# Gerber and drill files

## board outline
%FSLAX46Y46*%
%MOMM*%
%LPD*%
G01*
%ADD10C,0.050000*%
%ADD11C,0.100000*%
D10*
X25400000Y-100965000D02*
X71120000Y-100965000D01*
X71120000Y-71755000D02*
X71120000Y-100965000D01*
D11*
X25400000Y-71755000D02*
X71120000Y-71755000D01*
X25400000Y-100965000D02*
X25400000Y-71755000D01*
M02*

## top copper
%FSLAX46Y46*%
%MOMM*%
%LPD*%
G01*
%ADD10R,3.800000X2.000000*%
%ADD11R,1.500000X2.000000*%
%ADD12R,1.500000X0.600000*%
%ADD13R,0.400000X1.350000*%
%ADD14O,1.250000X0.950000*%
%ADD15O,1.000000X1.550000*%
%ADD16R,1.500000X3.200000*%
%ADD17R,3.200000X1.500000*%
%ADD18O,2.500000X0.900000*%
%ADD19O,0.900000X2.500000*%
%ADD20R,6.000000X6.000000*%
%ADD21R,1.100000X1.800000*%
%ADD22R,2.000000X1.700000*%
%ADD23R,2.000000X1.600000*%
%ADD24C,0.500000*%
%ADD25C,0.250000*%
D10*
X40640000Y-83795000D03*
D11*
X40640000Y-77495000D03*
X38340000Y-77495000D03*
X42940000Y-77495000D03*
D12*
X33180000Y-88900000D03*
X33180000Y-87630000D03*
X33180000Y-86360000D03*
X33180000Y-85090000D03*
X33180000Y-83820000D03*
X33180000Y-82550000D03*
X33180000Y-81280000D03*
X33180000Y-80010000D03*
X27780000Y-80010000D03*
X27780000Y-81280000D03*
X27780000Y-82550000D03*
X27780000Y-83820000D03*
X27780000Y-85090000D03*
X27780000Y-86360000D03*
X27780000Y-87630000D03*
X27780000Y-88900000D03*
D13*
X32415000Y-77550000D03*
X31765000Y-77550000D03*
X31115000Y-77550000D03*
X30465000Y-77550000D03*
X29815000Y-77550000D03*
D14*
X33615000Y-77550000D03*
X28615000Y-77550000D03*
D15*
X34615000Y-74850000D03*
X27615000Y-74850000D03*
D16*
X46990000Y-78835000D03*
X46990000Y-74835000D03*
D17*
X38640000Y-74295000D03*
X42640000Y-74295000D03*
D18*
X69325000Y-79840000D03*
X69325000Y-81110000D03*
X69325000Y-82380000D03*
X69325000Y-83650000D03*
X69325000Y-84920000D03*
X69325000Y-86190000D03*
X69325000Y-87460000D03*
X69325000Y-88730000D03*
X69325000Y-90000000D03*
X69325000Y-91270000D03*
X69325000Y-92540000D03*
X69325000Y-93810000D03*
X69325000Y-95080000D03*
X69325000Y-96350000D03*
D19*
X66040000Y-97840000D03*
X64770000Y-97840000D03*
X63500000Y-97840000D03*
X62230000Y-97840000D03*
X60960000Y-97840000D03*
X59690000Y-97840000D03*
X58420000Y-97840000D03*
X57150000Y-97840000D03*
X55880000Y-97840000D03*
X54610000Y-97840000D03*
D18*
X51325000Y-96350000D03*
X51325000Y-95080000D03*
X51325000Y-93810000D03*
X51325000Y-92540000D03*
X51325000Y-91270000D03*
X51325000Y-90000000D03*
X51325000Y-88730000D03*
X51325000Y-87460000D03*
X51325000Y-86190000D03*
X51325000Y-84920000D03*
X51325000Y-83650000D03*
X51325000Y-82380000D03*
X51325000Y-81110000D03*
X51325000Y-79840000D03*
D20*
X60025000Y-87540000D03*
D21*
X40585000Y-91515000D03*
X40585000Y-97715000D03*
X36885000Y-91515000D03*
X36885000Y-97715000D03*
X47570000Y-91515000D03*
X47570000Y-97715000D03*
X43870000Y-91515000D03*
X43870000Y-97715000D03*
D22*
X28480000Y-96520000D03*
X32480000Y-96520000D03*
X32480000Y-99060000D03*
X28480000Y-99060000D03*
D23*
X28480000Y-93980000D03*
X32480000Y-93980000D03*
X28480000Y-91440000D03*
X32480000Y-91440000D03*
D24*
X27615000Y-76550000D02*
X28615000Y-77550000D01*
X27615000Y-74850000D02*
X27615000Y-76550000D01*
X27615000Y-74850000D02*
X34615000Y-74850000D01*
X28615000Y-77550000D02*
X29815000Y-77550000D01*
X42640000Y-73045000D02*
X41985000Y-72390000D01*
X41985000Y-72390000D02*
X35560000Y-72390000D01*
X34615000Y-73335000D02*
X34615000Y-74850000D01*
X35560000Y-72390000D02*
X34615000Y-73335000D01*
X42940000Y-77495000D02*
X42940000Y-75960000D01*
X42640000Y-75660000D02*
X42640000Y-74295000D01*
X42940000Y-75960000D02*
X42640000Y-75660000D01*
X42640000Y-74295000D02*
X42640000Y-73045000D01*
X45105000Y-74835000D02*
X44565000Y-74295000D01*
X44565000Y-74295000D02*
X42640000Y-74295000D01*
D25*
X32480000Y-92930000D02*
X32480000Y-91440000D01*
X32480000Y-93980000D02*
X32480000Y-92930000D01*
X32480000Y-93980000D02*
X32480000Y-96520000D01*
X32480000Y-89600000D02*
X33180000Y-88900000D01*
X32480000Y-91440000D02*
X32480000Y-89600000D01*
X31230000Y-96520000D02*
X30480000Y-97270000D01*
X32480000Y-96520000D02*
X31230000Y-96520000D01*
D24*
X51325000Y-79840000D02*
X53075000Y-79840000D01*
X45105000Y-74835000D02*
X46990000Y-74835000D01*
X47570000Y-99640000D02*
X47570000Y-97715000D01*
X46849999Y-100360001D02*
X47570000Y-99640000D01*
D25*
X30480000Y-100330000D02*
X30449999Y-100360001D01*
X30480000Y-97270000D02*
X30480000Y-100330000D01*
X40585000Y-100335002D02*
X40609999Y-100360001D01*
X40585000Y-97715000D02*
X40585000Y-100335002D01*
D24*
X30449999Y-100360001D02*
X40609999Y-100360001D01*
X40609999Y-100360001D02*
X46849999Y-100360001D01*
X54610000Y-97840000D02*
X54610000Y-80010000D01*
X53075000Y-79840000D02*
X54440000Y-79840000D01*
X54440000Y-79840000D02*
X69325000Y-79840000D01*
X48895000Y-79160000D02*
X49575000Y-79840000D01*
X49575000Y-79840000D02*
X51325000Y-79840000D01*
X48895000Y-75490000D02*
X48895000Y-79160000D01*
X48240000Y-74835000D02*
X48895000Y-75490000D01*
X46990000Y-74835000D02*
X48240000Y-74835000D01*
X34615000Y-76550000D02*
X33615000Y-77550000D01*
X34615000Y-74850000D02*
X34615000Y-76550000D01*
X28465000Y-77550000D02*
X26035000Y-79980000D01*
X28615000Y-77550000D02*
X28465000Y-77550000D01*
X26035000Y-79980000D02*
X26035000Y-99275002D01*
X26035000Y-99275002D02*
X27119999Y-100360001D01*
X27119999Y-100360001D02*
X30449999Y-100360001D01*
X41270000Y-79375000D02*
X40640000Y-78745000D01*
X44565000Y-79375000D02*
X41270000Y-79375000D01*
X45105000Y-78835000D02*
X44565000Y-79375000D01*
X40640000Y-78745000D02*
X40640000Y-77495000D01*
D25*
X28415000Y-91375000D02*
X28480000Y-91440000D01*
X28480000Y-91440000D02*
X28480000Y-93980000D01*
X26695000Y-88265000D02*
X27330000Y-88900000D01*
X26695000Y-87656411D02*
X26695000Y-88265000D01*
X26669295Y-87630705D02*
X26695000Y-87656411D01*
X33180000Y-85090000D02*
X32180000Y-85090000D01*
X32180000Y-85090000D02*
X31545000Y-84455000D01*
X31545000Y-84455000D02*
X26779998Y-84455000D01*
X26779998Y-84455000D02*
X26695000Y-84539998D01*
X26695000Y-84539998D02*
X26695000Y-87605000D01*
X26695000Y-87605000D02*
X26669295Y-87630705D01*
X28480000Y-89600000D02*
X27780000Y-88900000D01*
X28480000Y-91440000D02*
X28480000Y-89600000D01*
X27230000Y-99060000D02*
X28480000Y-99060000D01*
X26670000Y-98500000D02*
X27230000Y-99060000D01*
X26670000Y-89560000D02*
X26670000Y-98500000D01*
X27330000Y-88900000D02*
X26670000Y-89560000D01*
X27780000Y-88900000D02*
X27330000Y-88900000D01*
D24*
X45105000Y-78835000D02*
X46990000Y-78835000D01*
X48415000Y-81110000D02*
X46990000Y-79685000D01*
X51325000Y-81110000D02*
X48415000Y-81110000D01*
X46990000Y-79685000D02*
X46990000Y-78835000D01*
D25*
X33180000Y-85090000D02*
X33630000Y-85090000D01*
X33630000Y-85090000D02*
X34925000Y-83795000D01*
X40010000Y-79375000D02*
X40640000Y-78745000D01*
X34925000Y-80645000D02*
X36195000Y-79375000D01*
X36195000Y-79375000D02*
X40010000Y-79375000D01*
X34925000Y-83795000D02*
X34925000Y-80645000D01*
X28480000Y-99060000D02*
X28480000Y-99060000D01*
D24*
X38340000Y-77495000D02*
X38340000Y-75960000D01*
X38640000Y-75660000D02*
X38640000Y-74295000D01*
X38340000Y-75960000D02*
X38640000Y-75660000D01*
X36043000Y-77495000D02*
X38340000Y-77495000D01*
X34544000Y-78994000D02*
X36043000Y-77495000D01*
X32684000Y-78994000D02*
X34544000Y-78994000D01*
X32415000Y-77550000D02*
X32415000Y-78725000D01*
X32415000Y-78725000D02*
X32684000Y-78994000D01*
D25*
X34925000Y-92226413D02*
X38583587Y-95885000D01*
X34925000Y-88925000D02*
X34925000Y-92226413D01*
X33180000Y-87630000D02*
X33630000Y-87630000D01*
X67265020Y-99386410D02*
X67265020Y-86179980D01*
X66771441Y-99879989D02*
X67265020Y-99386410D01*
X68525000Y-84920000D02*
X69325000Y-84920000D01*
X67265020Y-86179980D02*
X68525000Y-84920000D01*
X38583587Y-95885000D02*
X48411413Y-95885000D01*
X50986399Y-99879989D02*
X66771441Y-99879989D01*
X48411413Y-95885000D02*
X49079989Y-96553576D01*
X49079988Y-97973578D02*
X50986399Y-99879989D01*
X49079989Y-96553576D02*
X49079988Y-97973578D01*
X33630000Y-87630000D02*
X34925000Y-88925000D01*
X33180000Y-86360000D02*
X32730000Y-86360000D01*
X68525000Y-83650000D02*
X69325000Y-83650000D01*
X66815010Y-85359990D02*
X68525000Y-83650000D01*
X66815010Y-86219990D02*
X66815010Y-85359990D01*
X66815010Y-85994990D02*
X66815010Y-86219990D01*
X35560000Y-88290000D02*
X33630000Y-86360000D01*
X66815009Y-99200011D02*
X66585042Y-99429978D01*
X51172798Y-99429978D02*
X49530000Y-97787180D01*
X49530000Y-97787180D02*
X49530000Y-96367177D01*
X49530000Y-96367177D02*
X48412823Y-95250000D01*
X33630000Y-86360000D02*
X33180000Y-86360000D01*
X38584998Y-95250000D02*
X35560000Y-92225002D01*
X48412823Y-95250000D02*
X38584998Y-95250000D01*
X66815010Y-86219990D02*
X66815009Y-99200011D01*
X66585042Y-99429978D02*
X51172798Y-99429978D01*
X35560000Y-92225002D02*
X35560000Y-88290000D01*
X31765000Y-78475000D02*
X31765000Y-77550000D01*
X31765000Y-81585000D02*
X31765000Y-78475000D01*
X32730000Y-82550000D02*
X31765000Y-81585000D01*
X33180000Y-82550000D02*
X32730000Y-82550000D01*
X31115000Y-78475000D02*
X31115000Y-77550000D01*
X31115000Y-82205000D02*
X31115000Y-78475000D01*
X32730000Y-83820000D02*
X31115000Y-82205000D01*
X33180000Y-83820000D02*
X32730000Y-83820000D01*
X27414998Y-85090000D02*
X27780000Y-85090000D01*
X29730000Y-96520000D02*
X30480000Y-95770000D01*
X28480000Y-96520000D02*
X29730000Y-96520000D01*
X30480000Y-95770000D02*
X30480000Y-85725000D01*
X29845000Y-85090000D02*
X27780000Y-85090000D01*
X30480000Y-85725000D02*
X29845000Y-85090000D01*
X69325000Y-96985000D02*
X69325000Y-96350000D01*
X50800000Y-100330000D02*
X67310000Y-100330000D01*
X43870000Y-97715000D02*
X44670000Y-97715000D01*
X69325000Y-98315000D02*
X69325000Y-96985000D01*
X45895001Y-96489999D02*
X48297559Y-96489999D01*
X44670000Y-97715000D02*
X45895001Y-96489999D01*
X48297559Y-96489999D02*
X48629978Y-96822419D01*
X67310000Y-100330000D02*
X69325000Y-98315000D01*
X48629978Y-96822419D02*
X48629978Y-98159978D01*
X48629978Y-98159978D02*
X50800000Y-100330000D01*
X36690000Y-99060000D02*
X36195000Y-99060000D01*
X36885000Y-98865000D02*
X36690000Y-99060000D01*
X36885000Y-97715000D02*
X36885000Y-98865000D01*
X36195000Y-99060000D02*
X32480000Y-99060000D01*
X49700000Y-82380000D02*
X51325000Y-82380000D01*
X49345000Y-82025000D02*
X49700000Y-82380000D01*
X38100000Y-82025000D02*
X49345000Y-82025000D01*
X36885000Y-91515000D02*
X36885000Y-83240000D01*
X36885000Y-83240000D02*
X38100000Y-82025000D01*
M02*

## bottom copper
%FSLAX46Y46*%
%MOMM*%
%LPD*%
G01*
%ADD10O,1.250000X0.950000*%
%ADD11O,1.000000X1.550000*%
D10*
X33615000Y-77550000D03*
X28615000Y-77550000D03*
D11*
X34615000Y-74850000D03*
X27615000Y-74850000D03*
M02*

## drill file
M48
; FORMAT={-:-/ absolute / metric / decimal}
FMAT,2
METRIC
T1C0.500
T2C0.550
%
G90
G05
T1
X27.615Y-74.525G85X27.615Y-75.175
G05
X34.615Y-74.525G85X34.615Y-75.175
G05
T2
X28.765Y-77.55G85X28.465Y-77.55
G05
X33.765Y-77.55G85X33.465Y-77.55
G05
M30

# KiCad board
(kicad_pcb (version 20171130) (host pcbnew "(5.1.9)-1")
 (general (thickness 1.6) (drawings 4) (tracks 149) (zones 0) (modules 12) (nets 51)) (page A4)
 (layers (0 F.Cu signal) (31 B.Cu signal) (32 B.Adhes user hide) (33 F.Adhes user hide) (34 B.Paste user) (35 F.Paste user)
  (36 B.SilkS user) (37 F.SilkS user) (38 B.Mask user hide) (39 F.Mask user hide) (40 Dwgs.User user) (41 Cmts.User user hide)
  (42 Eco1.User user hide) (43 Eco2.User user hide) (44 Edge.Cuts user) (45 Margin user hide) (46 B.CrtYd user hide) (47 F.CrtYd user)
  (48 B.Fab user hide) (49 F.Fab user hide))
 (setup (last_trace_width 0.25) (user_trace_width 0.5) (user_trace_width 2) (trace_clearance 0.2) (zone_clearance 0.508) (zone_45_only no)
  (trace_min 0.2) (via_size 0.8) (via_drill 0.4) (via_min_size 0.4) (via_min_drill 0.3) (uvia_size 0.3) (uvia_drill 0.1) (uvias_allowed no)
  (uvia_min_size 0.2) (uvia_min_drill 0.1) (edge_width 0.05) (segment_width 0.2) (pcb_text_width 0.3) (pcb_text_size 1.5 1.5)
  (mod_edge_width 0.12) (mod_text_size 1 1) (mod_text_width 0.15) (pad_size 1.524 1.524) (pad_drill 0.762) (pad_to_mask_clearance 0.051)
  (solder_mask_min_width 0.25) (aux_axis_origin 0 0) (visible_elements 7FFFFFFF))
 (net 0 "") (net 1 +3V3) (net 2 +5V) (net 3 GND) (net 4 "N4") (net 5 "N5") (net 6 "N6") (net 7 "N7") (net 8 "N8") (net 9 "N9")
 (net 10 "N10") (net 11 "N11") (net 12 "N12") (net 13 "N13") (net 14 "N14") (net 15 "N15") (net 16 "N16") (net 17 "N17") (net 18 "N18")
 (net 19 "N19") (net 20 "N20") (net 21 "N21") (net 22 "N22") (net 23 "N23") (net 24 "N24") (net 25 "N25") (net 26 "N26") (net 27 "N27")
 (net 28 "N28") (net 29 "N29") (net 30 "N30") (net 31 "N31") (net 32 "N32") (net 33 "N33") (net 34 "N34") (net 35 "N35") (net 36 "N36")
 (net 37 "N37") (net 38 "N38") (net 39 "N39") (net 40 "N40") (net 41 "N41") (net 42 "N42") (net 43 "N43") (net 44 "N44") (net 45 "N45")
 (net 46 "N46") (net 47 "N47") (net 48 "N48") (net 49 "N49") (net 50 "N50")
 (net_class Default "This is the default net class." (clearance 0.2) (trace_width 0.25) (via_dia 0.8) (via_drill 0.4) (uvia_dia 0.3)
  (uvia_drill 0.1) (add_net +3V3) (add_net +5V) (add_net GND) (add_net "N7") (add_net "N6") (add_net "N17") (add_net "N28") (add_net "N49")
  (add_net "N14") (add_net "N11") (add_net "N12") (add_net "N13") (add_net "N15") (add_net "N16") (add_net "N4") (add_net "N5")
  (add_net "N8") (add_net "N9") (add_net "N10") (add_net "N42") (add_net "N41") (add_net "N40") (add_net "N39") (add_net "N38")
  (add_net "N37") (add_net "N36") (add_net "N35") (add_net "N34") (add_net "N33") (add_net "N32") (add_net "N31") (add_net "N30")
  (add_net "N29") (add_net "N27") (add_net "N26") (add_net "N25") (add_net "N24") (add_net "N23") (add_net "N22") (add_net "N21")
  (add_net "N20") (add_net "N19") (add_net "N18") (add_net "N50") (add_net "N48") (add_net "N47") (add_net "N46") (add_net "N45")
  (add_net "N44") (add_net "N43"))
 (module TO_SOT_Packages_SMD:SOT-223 (layer F.Cu) (at 40.64 80.645 270)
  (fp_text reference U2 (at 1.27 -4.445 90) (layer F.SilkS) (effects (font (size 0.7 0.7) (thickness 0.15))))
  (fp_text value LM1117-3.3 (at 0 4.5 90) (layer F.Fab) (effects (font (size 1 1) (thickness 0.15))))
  (pad 4 smd rect (at 3.15 0 270) (size 2 3.8) (layers F.Cu F.Paste F.Mask))
  (pad 2 smd rect (at -3.15 0 270) (size 2 1.5) (layers F.Cu F.Paste F.Mask) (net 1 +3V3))
  (pad 3 smd rect (at -3.15 2.3 270) (size 2 1.5) (layers F.Cu F.Paste F.Mask) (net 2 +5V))
  (pad 1 smd rect (at -3.15 -2.3 270) (size 2 1.5) (layers F.Cu F.Paste F.Mask) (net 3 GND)))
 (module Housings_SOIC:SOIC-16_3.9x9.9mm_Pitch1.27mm (layer F.Cu) (at 30.48 84.455 180)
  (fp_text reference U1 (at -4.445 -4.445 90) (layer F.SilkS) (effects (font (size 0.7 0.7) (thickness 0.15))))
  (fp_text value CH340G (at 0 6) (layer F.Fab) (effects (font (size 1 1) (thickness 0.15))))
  (pad 1 smd rect (at -2.7 -4.445 180) (size 1.5 0.6) (layers F.Cu F.Paste F.Mask) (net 3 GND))
  (pad 2 smd rect (at -2.7 -3.175 180) (size 1.5 0.6) (layers F.Cu F.Paste F.Mask) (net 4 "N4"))
  (pad 3 smd rect (at -2.7 -1.905 180) (size 1.5 0.6) (layers F.Cu F.Paste F.Mask) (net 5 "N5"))
  (pad 4 smd rect (at -2.7 -0.635 180) (size 1.5 0.6) (layers F.Cu F.Paste F.Mask) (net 1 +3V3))
  (pad 5 smd rect (at -2.7 0.635 180) (size 1.5 0.6) (layers F.Cu F.Paste F.Mask) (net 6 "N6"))
  (pad 6 smd rect (at -2.7 1.905 180) (size 1.5 0.6) (layers F.Cu F.Paste F.Mask) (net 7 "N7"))
  (pad 7 smd rect (at -2.7 3.175 180) (size 1.5 0.6) (layers F.Cu F.Paste F.Mask) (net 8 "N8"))
  (pad 8 smd rect (at -2.7 4.445 180) (size 1.5 0.6) (layers F.Cu F.Paste F.Mask) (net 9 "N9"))
  (pad 9 smd rect (at 2.7 4.445 180) (size 1.5 0.6) (layers F.Cu F.Paste F.Mask) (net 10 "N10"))
  (pad 10 smd rect (at 2.7 3.175 180) (size 1.5 0.6) (layers F.Cu F.Paste F.Mask) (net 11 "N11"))
  (pad 11 smd rect (at 2.7 1.905 180) (size 1.5 0.6) (layers F.Cu F.Paste F.Mask) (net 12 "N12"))
  (pad 12 smd rect (at 2.7 0.635 180) (size 1.5 0.6) (layers F.Cu F.Paste F.Mask) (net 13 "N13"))
  (pad 13 smd rect (at 2.7 -0.635 180) (size 1.5 0.6) (layers F.Cu F.Paste F.Mask) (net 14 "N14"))
  (pad 14 smd rect (at 2.7 -1.905 180) (size 1.5 0.6) (layers F.Cu F.Paste F.Mask) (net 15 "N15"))
  (pad 15 smd rect (at 2.7 -3.175 180) (size 1.5 0.6) (layers F.Cu F.Paste F.Mask) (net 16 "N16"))
  (pad 16 smd rect (at 2.7 -4.445 180) (size 1.5 0.6) (layers F.Cu F.Paste F.Mask) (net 1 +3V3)))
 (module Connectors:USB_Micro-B (layer F.Cu) (at 31.115 76.2 180)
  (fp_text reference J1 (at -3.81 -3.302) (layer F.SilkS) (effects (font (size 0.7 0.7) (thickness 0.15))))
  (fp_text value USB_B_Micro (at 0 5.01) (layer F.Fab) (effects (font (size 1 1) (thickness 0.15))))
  (pad 1 smd rect (at -1.3 -1.35 270) (size 1.35 0.4) (layers F.Cu F.Paste F.Mask) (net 2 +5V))
  (pad 2 smd rect (at -0.65 -1.35 270) (size 1.35 0.4) (layers F.Cu F.Paste F.Mask) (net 7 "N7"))
  (pad 3 smd rect (at 0 -1.35 270) (size 1.35 0.4) (layers F.Cu F.Paste F.Mask) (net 6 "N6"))
  (pad 4 smd rect (at 0.65 -1.35 270) (size 1.35 0.4) (layers F.Cu F.Paste F.Mask) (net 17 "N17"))
  (pad 5 smd rect (at 1.3 -1.35 270) (size 1.35 0.4) (layers F.Cu F.Paste F.Mask) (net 3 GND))
  (pad 6 thru_hole oval (at -2.5 -1.35 270) (size 0.95 1.25) (drill oval 0.55 0.85) (layers *.Cu *.Mask) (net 3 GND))
  (pad 6 thru_hole oval (at 2.5 -1.35 270) (size 0.95 1.25) (drill oval 0.55 0.85) (layers *.Cu *.Mask) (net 3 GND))
  (pad 6 thru_hole oval (at -3.5 1.35 270) (size 1.55 1) (drill oval 1.15 0.5) (layers *.Cu *.Mask) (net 3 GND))
  (pad 6 thru_hole oval (at 3.5 1.35 270) (size 1.55 1) (drill oval 1.15 0.5) (layers *.Cu *.Mask) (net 3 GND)))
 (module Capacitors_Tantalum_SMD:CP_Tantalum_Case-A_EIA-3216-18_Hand (layer F.Cu) (at 46.99 76.835 90)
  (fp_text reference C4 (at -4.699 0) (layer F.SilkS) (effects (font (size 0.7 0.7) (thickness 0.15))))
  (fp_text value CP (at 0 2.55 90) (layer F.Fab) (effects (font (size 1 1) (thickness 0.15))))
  (pad 1 smd rect (at -2 0 90) (size 3.2 1.5) (layers F.Cu F.Paste F.Mask) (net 1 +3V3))
  (pad 2 smd rect (at 2 0 90) (size 3.2 1.5) (layers F.Cu F.Paste F.Mask) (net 3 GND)))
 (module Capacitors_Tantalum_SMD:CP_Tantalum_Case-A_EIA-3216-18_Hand (layer F.Cu) (at 40.64 74.295)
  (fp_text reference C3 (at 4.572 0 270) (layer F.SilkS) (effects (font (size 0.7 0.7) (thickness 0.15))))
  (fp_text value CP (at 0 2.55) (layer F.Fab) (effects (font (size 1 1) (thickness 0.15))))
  (pad 1 smd rect (at -2 0) (size 3.2 1.5) (layers F.Cu F.Paste F.Mask) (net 2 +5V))
  (pad 2 smd rect (at 2 0) (size 3.2 1.5) (layers F.Cu F.Paste F.Mask) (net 3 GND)))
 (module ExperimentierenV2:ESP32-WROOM (layer F.Cu) (at 60.325 85.09 180)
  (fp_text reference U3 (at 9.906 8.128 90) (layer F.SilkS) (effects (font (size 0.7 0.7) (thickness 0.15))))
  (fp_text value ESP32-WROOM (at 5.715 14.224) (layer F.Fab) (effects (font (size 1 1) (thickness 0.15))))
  (pad 38 smd oval (at -9 5.25 180) (size 2.5 0.9) (layers F.Cu F.Paste F.Mask) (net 3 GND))
  (pad 37 smd oval (at -9 3.98 180) (size 2.5 0.9) (layers F.Cu F.Paste F.Mask) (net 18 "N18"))
  (pad 36 smd oval (at -9 2.71 180) (size 2.5 0.9) (layers F.Cu F.Paste F.Mask) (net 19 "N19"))
  (pad 35 smd oval (at -9 1.44 180) (size 2.5 0.9) (layers F.Cu F.Paste F.Mask) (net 5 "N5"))
  (pad 34 smd oval (at -9 0.17 180) (size 2.5 0.9) (layers F.Cu F.Paste F.Mask) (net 4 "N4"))
  (pad 33 smd oval (at -9 -1.1 180) (size 2.5 0.9) (layers F.Cu F.Paste F.Mask) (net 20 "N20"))
  (pad 32 smd oval (at -9 -2.37 180) (size 2.5 0.9) (layers F.Cu F.Paste F.Mask) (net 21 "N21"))
  (pad 31 smd oval (at -9 -3.64 180) (size 2.5 0.9) (layers F.Cu F.Paste F.Mask) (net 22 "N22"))
  (pad 30 smd oval (at -9 -4.91 180) (size 2.5 0.9) (layers F.Cu F.Paste F.Mask) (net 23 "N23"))
  (pad 29 smd oval (at -9 -6.18 180) (size 2.5 0.9) (layers F.Cu F.Paste F.Mask) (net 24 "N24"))
  (pad 28 smd oval (at -9 -7.45 180) (size 2.5 0.9) (layers F.Cu F.Paste F.Mask) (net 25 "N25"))
  (pad 27 smd oval (at -9 -8.72 180) (size 2.5 0.9) (layers F.Cu F.Paste F.Mask) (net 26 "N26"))
  (pad 26 smd oval (at -9 -9.99 180) (size 2.5 0.9) (layers F.Cu F.Paste F.Mask) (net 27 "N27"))
  (pad 25 smd oval (at -9 -11.26 180) (size 2.5 0.9) (layers F.Cu F.Paste F.Mask) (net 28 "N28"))
  (pad 24 smd oval (at -5.715 -12.75 180) (size 0.9 2.5) (layers F.Cu F.Paste F.Mask) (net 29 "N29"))
  (pad 23 smd oval (at -4.445 -12.75 180) (size 0.9 2.5) (layers F.Cu F.Paste F.Mask) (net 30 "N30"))
  (pad 22 smd oval (at -3.175 -12.75 180) (size 0.9 2.5) (layers F.Cu F.Paste F.Mask) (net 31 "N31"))
  (pad 21 smd oval (at -1.905 -12.75 180) (size 0.9 2.5) (layers F.Cu F.Paste F.Mask) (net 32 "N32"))
  (pad 20 smd oval (at -0.635 -12.75 180) (size 0.9 2.5) (layers F.Cu F.Paste F.Mask) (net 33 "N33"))
  (pad 19 smd oval (at 0.635 -12.75 180) (size 0.9 2.5) (layers F.Cu F.Paste F.Mask) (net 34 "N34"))
  (pad 18 smd oval (at 1.905 -12.75 180) (size 0.9 2.5) (layers F.Cu F.Paste F.Mask) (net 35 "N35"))
  (pad 17 smd oval (at 3.175 -12.75 180) (size 0.9 2.5) (layers F.Cu F.Paste F.Mask) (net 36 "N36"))
  (pad 16 smd oval (at 4.445 -12.75 180) (size 0.9 2.5) (layers F.Cu F.Paste F.Mask) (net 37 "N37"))
  (pad 15 smd oval (at 5.715 -12.75 180) (size 0.9 2.5) (layers F.Cu F.Paste F.Mask) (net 3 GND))
  (pad 14 smd oval (at 9 -11.26 180) (size 2.5 0.9) (layers F.Cu F.Paste F.Mask) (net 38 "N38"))
  (pad 13 smd oval (at 9 -9.99 180) (size 2.5 0.9) (layers F.Cu F.Paste F.Mask) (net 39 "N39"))
  (pad 12 smd oval (at 9 -8.72 180) (size 2.5 0.9) (layers F.Cu F.Paste F.Mask) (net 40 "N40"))
  (pad 11 smd oval (at 9 -7.45 180) (size 2.5 0.9) (layers F.Cu F.Paste F.Mask) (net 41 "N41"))
  (pad 10 smd oval (at 9 -6.18 180) (size 2.5 0.9) (layers F.Cu F.Paste F.Mask) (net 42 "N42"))
  (pad 9 smd oval (at 9 -4.91 180) (size 2.5 0.9) (layers F.Cu F.Paste F.Mask) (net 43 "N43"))
  (pad 8 smd oval (at 9 -3.64 180) (size 2.5 0.9) (layers F.Cu F.Paste F.Mask) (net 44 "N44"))
  (pad 7 smd oval (at 9 -2.37 180) (size 2.5 0.9) (layers F.Cu F.Paste F.Mask) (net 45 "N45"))
  (pad 6 smd oval (at 9 -1.1 180) (size 2.5 0.9) (layers F.Cu F.Paste F.Mask) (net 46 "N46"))
  (pad 5 smd oval (at 9 0.17 180) (size 2.5 0.9) (layers F.Cu F.Paste F.Mask) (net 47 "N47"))
  (pad 4 smd oval (at 9 1.44 180) (size 2.5 0.9) (layers F.Cu F.Paste F.Mask) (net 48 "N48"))
  (pad 3 smd oval (at 9 2.71 180) (size 2.5 0.9) (layers F.Cu F.Paste F.Mask) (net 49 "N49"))
  (pad 2 smd oval (at 9 3.98 180) (size 2.5 0.9) (layers F.Cu F.Paste F.Mask) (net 1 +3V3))
  (pad 1 smd oval (at 9 5.25 180) (size 2.5 0.9) (layers F.Cu F.Paste F.Mask) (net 3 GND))
  (pad 39 smd rect (at 0.3 -2.45 180) (size 6 6) (layers F.Cu F.Paste F.Mask) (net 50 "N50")))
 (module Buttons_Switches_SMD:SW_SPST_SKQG (layer F.Cu) (at 38.735 94.615 270)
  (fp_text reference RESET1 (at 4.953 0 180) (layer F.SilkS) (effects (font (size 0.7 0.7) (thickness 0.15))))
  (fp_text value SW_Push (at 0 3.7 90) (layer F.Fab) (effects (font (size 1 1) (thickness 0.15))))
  (pad 1 smd rect (at -3.1 -1.85 270) (size 1.8 1.1) (layers F.Cu F.Paste F.Mask) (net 3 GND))
  (pad 1 smd rect (at 3.1 -1.85 270) (size 1.8 1.1) (layers F.Cu F.Paste F.Mask) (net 3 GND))
  (pad 2 smd rect (at -3.1 1.85 270) (size 1.8 1.1) (layers F.Cu F.Paste F.Mask) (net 49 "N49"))
  (pad 2 smd rect (at 3.1 1.85 270) (size 1.8 1.1) (layers F.Cu F.Paste F.Mask) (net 49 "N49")))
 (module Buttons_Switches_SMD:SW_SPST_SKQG (layer F.Cu) (at 45.72 94.615 270)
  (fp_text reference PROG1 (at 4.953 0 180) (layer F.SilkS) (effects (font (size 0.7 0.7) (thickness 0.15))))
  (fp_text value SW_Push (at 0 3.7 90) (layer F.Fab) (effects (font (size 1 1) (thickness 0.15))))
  (pad 1 smd rect (at -3.1 -1.85 270) (size 1.8 1.1) (layers F.Cu F.Paste F.Mask) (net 3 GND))
  (pad 1 smd rect (at 3.1 -1.85 270) (size 1.8 1.1) (layers F.Cu F.Paste F.Mask) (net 3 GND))
  (pad 2 smd rect (at -3.1 1.85 270) (size 1.8 1.1) (layers F.Cu F.Paste F.Mask) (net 28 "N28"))
  (pad 2 smd rect (at 3.1 1.85 270) (size 1.8 1.1) (layers F.Cu F.Paste F.Mask) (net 28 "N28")))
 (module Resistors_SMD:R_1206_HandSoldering (layer F.Cu) (at 30.48 96.52)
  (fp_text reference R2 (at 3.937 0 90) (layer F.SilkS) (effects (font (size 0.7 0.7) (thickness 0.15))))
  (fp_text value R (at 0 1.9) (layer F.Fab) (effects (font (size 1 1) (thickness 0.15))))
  (pad 1 smd rect (at -2 0) (size 2 1.7) (layers F.Cu F.Paste F.Mask) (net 14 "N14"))
  (pad 2 smd rect (at 2 0) (size 2 1.7) (layers F.Cu F.Paste F.Mask) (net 3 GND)))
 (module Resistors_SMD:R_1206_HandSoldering (layer F.Cu) (at 30.48 99.06 180)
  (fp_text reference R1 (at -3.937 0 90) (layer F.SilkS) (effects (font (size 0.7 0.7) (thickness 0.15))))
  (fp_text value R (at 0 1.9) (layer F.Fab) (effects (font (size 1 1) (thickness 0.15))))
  (pad 1 smd rect (at -2 0 180) (size 2 1.7) (layers F.Cu F.Paste F.Mask) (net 49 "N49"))
  (pad 2 smd rect (at 2 0 180) (size 2 1.7) (layers F.Cu F.Paste F.Mask) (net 1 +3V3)))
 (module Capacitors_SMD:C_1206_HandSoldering (layer F.Cu) (at 30.48 93.98)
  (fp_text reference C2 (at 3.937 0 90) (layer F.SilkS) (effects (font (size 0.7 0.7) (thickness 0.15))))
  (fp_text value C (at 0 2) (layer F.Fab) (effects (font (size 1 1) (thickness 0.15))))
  (pad 1 smd rect (at -2 0) (size 2 1.6) (layers F.Cu F.Paste F.Mask) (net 1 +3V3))
  (pad 2 smd rect (at 2 0) (size 2 1.6) (layers F.Cu F.Paste F.Mask) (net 3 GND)))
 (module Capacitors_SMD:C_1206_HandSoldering (layer F.Cu) (at 30.48 91.44)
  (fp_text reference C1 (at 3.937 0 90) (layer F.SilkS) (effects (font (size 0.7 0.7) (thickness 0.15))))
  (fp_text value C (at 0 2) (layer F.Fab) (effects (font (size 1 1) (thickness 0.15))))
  (pad 1 smd rect (at -2 0) (size 2 1.6) (layers F.Cu F.Paste F.Mask) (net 1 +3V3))
  (pad 2 smd rect (at 2 0) (size 2 1.6) (layers F.Cu F.Paste F.Mask) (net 3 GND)))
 (gr_line (start 25.4 100.965) (end 71.12 100.965) (layer Edge.Cuts) (width 0.05))
 (gr_line (start 71.12 71.755) (end 71.12 100.965) (layer Edge.Cuts) (width 0.05))
 (gr_line (start 25.4 71.755) (end 71.12 71.755) (layer Edge.Cuts) (width 0.1))
 (gr_line (start 25.4 100.965) (end 25.4 71.755) (layer Edge.Cuts) (width 0.1))
 (segment (start 27.615 76.55) (end 28.615 77.55) (width 0.5) (layer F.Cu) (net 3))
 (segment (start 27.615 74.85) (end 27.615 76.55) (width 0.5) (layer F.Cu) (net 3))
 (segment (start 27.615 74.85) (end 34.615 74.85) (width 0.5) (layer F.Cu) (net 3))
 (segment (start 28.615 77.55) (end 29.815 77.55) (width 0.5) (layer F.Cu) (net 3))
 (segment (start 42.64 73.045) (end 41.985 72.39) (width 0.5) (layer F.Cu) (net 3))
 (segment (start 41.985 72.39) (end 35.56 72.39) (width 0.5) (layer F.Cu) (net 3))
 (segment (start 34.615 73.335) (end 34.615 74.85) (width 0.5) (layer F.Cu) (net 3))
 (segment (start 35.56 72.39) (end 34.615 73.335) (width 0.5) (layer F.Cu) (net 3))
 (segment (start 42.94 77.495) (end 42.94 75.96) (width 0.5) (layer F.Cu) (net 3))
 (segment (start 42.64 75.66) (end 42.64 74.295) (width 0.5) (layer F.Cu) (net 3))
 (segment (start 42.94 75.96) (end 42.64 75.66) (width 0.5) (layer F.Cu) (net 3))
 (segment (start 42.64 74.295) (end 42.64 73.045) (width 0.5) (layer F.Cu) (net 3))
 (segment (start 45.105 74.835) (end 44.565 74.295) (width 0.5) (layer F.Cu) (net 3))
 (segment (start 44.565 74.295) (end 42.64 74.295) (width 0.5) (layer F.Cu) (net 3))
 (segment (start 32.48 92.93) (end 32.48 91.44) (width 0.25) (layer F.Cu) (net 3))
 (segment (start 32.48 93.98) (end 32.48 92.93) (width 0.25) (layer F.Cu) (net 3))
 (segment (start 32.48 93.98) (end 32.48 96.52) (width 0.25) (layer F.Cu) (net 3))
 (segment (start 32.48 89.6) (end 33.18 88.9) (width 0.25) (layer F.Cu) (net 3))
 (segment (start 32.48 91.44) (end 32.48 89.6) (width 0.25) (layer F.Cu) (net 3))
 (segment (start 31.23 96.52) (end 30.48 97.27) (width 0.25) (layer F.Cu) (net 3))
 (segment (start 32.48 96.52) (end 31.23 96.52) (width 0.25) (layer F.Cu) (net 3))
 (segment (start 51.325 79.84) (end 53.075 79.84) (width 0.5) (layer F.Cu) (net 3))
 (segment (start 45.105 74.835) (end 46.99 74.835) (width 0.5) (layer F.Cu) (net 3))
 (segment (start 47.57 99.64) (end 47.57 97.715) (width 0.5) (layer F.Cu) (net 3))
 (segment (start 46.849999 100.360001) (end 47.57 99.64) (width 0.5) (layer F.Cu) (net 3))
 (segment (start 30.48 100.33) (end 30.449999 100.360001) (width 0.25) (layer F.Cu) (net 3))
 (segment (start 30.48 97.27) (end 30.48 100.33) (width 0.25) (layer F.Cu) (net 3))
 (segment (start 40.585 100.335002) (end 40.609999 100.360001) (width 0.25) (layer F.Cu) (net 3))
 (segment (start 40.585 97.715) (end 40.585 100.335002) (width 0.25) (layer F.Cu) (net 3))
 (segment (start 30.449999 100.360001) (end 40.609999 100.360001) (width 0.5) (layer F.Cu) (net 3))
 (segment (start 40.609999 100.360001) (end 46.849999 100.360001) (width 0.5) (layer F.Cu) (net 3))
 (segment (start 54.61 97.84) (end 54.61 80.01) (width 0.5) (layer F.Cu) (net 3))
 (segment (start 53.075 79.84) (end 54.44 79.84) (width 0.5) (layer F.Cu) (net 3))
 (segment (start 54.44 79.84) (end 69.325 79.84) (width 0.5) (layer F.Cu) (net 3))
 (segment (start 48.895 79.16) (end 49.575 79.84) (width 0.5) (layer F.Cu) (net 3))
 (segment (start 49.575 79.84) (end 51.325 79.84) (width 0.5) (layer F.Cu) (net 3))
 (segment (start 48.895 75.49) (end 48.895 79.16) (width 0.5) (layer F.Cu) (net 3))
 (segment (start 48.24 74.835) (end 48.895 75.49) (width 0.5) (layer F.Cu) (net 3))
 (segment (start 46.99 74.835) (end 48.24 74.835) (width 0.5) (layer F.Cu) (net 3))
 (segment (start 34.615 76.55) (end 33.615 77.55) (width 0.5) (layer F.Cu) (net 3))
 (segment (start 34.615 74.85) (end 34.615 76.55) (width 0.5) (layer F.Cu) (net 3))
 (segment (start 28.465 77.55) (end 26.035 79.98) (width 0.5) (layer F.Cu) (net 3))
 (segment (start 28.615 77.55) (end 28.465 77.55) (width 0.5) (layer F.Cu) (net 3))
 (segment (start 26.035 79.98) (end 26.035 99.275002) (width 0.5) (layer F.Cu) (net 3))
 (segment (start 26.035 99.275002) (end 27.119999 100.360001) (width 0.5) (layer F.Cu) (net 3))
 (segment (start 27.119999 100.360001) (end 30.449999 100.360001) (width 0.5) (layer F.Cu) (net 3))
 (segment (start 41.27 79.375) (end 40.64 78.745) (width 0.5) (layer F.Cu) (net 1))
 (segment (start 44.565 79.375) (end 41.27 79.375) (width 0.5) (layer F.Cu) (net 1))
 (segment (start 45.105 78.835) (end 44.565 79.375) (width 0.5) (layer F.Cu) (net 1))
 (segment (start 40.64 78.745) (end 40.64 77.495) (width 0.5) (layer F.Cu) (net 1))
 (segment (start 28.415 91.375) (end 28.48 91.44) (width 0.25) (layer F.Cu) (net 1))
 (segment (start 28.48 91.44) (end 28.48 93.98) (width 0.25) (layer F.Cu) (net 1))
 (segment (start 26.695 88.265) (end 27.33 88.9) (width 0.25) (layer F.Cu) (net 1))
 (segment (start 26.695 87.656411) (end 26.695 88.265) (width 0.25) (layer F.Cu) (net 1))
 (segment (start 26.669295 87.630705) (end 26.695 87.656411) (width 0.25) (layer F.Cu) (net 1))
 (segment (start 33.18 85.09) (end 32.18 85.09) (width 0.25) (layer F.Cu) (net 1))
 (segment (start 32.18 85.09) (end 31.545 84.455) (width 0.25) (layer F.Cu) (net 1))
 (segment (start 31.545 84.455) (end 26.779998 84.455) (width 0.25) (layer F.Cu) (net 1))
 (segment (start 26.779998 84.455) (end 26.695 84.539998) (width 0.25) (layer F.Cu) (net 1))
 (segment (start 26.695 84.539998) (end 26.695 87.605) (width 0.25) (layer F.Cu) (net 1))
 (segment (start 26.695 87.605) (end 26.669295 87.630705) (width 0.25) (layer F.Cu) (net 1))
 (segment (start 28.48 89.6) (end 27.78 88.9) (width 0.25) (layer F.Cu) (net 1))
 (segment (start 28.48 91.44) (end 28.48 89.6) (width 0.25) (layer F.Cu) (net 1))
 (segment (start 27.23 99.06) (end 28.48 99.06) (width 0.25) (layer F.Cu) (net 1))
 (segment (start 26.67 98.5) (end 27.23 99.06) (width 0.25) (layer F.Cu) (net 1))
 (segment (start 26.67 89.56) (end 26.67 98.5) (width 0.25) (layer F.Cu) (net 1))
 (segment (start 27.33 88.9) (end 26.67 89.56) (width 0.25) (layer F.Cu) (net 1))
 (segment (start 27.78 88.9) (end 27.33 88.9) (width 0.25) (layer F.Cu) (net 1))
 (segment (start 45.105 78.835) (end 46.99 78.835) (width 0.5) (layer F.Cu) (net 1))
 (segment (start 48.415 81.11) (end 46.99 79.685) (width 0.5) (layer F.Cu) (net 1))
 (segment (start 51.325 81.11) (end 48.415 81.11) (width 0.5) (layer F.Cu) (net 1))
 (segment (start 46.99 79.685) (end 46.99 78.835) (width 0.5) (layer F.Cu) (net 1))
 (segment (start 33.18 85.09) (end 33.63 85.09) (width 0.25) (layer F.Cu) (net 1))
 (segment (start 33.63 85.09) (end 34.925 83.795) (width 0.25) (layer F.Cu) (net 1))
 (segment (start 40.01 79.375) (end 40.64 78.745) (width 0.25) (layer F.Cu) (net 1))
 (segment (start 34.925 80.645) (end 36.195 79.375) (width 0.25) (layer F.Cu) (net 1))
 (segment (start 36.195 79.375) (end 40.01 79.375) (width 0.25) (layer F.Cu) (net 1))
 (segment (start 34.925 83.795) (end 34.925 80.645) (width 0.25) (layer F.Cu) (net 1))
 (segment (start 28.48 99.06) (end 28.48 99.06) (width 0.25) (layer F.Cu) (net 1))
 (segment (start 38.34 77.495) (end 38.34 75.96) (width 0.5) (layer F.Cu) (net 2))
 (segment (start 38.64 75.66) (end 38.64 74.295) (width 0.5) (layer F.Cu) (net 2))
 (segment (start 38.34 75.96) (end 38.64 75.66) (width 0.5) (layer F.Cu) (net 2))
 (segment (start 36.043 77.495) (end 38.34 77.495) (width 0.5) (layer F.Cu) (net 2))
 (segment (start 34.544 78.994) (end 36.043 77.495) (width 0.5) (layer F.Cu) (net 2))
 (segment (start 32.684 78.994) (end 34.544 78.994) (width 0.5) (layer F.Cu) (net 2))
 (segment (start 32.415 77.55) (end 32.415 78.725) (width 0.5) (layer F.Cu) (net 2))
 (segment (start 32.415 78.725) (end 32.684 78.994) (width 0.5) (layer F.Cu) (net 2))
 (segment (start 34.925 92.226413) (end 38.583587 95.885) (width 0.25) (layer F.Cu) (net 4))
 (segment (start 34.925 88.925) (end 34.925 92.226413) (width 0.25) (layer F.Cu) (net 4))
 (segment (start 33.18 87.63) (end 33.63 87.63) (width 0.25) (layer F.Cu) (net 4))
 (segment (start 67.26502 99.38641) (end 67.26502 86.17998) (width 0.25) (layer F.Cu) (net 4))
 (segment (start 66.771441 99.879989) (end 67.26502 99.38641) (width 0.25) (layer F.Cu) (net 4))
 (segment (start 68.525 84.92) (end 69.325 84.92) (width 0.25) (layer F.Cu) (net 4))
 (segment (start 67.26502 86.17998) (end 68.525 84.92) (width 0.25) (layer F.Cu) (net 4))
 (segment (start 38.583587 95.885) (end 48.411413 95.885) (width 0.25) (layer F.Cu) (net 4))
 (segment (start 50.986399 99.879989) (end 66.771441 99.879989) (width 0.25) (layer F.Cu) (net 4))
 (segment (start 48.411413 95.885) (end 49.079989 96.553576) (width 0.25) (layer F.Cu) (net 4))
 (segment (start 49.079988 97.973578) (end 50.986399 99.879989) (width 0.25) (layer F.Cu) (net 4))
 (segment (start 49.079989 96.553576) (end 49.079988 97.973578) (width 0.25) (layer F.Cu) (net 4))
 (segment (start 33.63 87.63) (end 34.925 88.925) (width 0.25) (layer F.Cu) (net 4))
 (segment (start 33.18 86.36) (end 32.73 86.36) (width 0.25) (layer F.Cu) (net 5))
 (segment (start 68.525 83.65) (end 69.325 83.65) (width 0.25) (layer F.Cu) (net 5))
 (segment (start 66.81501 85.35999) (end 68.525 83.65) (width 0.25) (layer F.Cu) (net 5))
 (segment (start 66.81501 86.21999) (end 66.81501 85.35999) (width 0.25) (layer F.Cu) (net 5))
 (segment (start 66.81501 85.99499) (end 66.81501 86.21999) (width 0.25) (layer F.Cu) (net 5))
 (segment (start 35.56 88.29) (end 33.63 86.36) (width 0.25) (layer F.Cu) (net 5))
 (segment (start 66.815009 99.200011) (end 66.585042 99.429978) (width 0.25) (layer F.Cu) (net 5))
 (segment (start 51.172798 99.429978) (end 49.53 97.78718) (width 0.25) (layer F.Cu) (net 5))
 (segment (start 49.53 97.78718) (end 49.53 96.367177) (width 0.25) (layer F.Cu) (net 5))
 (segment (start 49.53 96.367177) (end 48.412823 95.25) (width 0.25) (layer F.Cu) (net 5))
 (segment (start 33.63 86.36) (end 33.18 86.36) (width 0.25) (layer F.Cu) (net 5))
 (segment (start 38.584998 95.25) (end 35.56 92.225002) (width 0.25) (layer F.Cu) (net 5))
 (segment (start 48.412823 95.25) (end 38.584998 95.25) (width 0.25) (layer F.Cu) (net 5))
 (segment (start 66.81501 86.21999) (end 66.815009 99.200011) (width 0.25) (layer F.Cu) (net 5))
 (segment (start 66.585042 99.429978) (end 51.172798 99.429978) (width 0.25) (layer F.Cu) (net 5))
 (segment (start 35.56 92.225002) (end 35.56 88.29) (width 0.25) (layer F.Cu) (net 5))
 (segment (start 31.765 78.475) (end 31.765 77.55) (width 0.25) (layer F.Cu) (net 7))
 (segment (start 31.765 81.585) (end 31.765 78.475) (width 0.25) (layer F.Cu) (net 7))
 (segment (start 32.73 82.55) (end 31.765 81.585) (width 0.25) (layer F.Cu) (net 7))
 (segment (start 33.18 82.55) (end 32.73 82.55) (width 0.25) (layer F.Cu) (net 7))
 (segment (start 31.115 78.475) (end 31.115 77.55) (width 0.25) (layer F.Cu) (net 6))
 (segment (start 31.115 82.205) (end 31.115 78.475) (width 0.25) (layer F.Cu) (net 6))
 (segment (start 32.73 83.82) (end 31.115 82.205) (width 0.25) (layer F.Cu) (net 6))
 (segment (start 33.18 83.82) (end 32.73 83.82) (width 0.25) (layer F.Cu) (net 6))
 (segment (start 27.414998 85.09) (end 27.78 85.09) (width 0.25) (layer F.Cu) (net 14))
 (segment (start 29.73 96.52) (end 30.48 95.77) (width 0.25) (layer F.Cu) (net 14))
 (segment (start 28.48 96.52) (end 29.73 96.52) (width 0.25) (layer F.Cu) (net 14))
 (segment (start 30.48 95.77) (end 30.48 85.725) (width 0.25) (layer F.Cu) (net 14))
 (segment (start 29.845 85.09) (end 27.78 85.09) (width 0.25) (layer F.Cu) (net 14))
 (segment (start 30.48 85.725) (end 29.845 85.09) (width 0.25) (layer F.Cu) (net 14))
 (segment (start 69.325 96.985) (end 69.325 96.35) (width 0.25) (layer F.Cu) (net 28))
 (segment (start 50.8 100.33) (end 67.31 100.33) (width 0.25) (layer F.Cu) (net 28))
 (segment (start 43.87 97.715) (end 44.67 97.715) (width 0.25) (layer F.Cu) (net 28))
 (segment (start 69.325 98.315) (end 69.325 96.985) (width 0.25) (layer F.Cu) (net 28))
 (segment (start 45.895001 96.489999) (end 48.297559 96.489999) (width 0.25) (layer F.Cu) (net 28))
 (segment (start 44.67 97.715) (end 45.895001 96.489999) (width 0.25) (layer F.Cu) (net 28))
 (segment (start 48.297559 96.489999) (end 48.629978 96.822419) (width 0.25) (layer F.Cu) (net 28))
 (segment (start 67.31 100.33) (end 69.325 98.315) (width 0.25) (layer F.Cu) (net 28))
 (segment (start 48.629978 96.822419) (end 48.629978 98.159978) (width 0.25) (layer F.Cu) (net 28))
 (segment (start 48.629978 98.159978) (end 50.8 100.33) (width 0.25) (layer F.Cu) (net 28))
 (segment (start 36.69 99.06) (end 36.195 99.06) (width 0.25) (layer F.Cu) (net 49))
 (segment (start 36.885 98.865) (end 36.69 99.06) (width 0.25) (layer F.Cu) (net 49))
 (segment (start 36.885 97.715) (end 36.885 98.865) (width 0.25) (layer F.Cu) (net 49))
 (segment (start 36.195 99.06) (end 32.48 99.06) (width 0.25) (layer F.Cu) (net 49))
 (segment (start 49.7 82.38) (end 51.325 82.38) (width 0.25) (layer F.Cu) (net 49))
 (segment (start 49.345 82.025) (end 49.7 82.38) (width 0.25) (layer F.Cu) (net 49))
 (segment (start 38.1 82.025) (end 49.345 82.025) (width 0.25) (layer F.Cu) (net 49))
 (segment (start 36.885 91.515) (end 36.885 83.24) (width 0.25) (layer F.Cu) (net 49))
 (segment (start 36.885 83.24) (end 38.1 82.025) (width 0.25) (layer F.Cu) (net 49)))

